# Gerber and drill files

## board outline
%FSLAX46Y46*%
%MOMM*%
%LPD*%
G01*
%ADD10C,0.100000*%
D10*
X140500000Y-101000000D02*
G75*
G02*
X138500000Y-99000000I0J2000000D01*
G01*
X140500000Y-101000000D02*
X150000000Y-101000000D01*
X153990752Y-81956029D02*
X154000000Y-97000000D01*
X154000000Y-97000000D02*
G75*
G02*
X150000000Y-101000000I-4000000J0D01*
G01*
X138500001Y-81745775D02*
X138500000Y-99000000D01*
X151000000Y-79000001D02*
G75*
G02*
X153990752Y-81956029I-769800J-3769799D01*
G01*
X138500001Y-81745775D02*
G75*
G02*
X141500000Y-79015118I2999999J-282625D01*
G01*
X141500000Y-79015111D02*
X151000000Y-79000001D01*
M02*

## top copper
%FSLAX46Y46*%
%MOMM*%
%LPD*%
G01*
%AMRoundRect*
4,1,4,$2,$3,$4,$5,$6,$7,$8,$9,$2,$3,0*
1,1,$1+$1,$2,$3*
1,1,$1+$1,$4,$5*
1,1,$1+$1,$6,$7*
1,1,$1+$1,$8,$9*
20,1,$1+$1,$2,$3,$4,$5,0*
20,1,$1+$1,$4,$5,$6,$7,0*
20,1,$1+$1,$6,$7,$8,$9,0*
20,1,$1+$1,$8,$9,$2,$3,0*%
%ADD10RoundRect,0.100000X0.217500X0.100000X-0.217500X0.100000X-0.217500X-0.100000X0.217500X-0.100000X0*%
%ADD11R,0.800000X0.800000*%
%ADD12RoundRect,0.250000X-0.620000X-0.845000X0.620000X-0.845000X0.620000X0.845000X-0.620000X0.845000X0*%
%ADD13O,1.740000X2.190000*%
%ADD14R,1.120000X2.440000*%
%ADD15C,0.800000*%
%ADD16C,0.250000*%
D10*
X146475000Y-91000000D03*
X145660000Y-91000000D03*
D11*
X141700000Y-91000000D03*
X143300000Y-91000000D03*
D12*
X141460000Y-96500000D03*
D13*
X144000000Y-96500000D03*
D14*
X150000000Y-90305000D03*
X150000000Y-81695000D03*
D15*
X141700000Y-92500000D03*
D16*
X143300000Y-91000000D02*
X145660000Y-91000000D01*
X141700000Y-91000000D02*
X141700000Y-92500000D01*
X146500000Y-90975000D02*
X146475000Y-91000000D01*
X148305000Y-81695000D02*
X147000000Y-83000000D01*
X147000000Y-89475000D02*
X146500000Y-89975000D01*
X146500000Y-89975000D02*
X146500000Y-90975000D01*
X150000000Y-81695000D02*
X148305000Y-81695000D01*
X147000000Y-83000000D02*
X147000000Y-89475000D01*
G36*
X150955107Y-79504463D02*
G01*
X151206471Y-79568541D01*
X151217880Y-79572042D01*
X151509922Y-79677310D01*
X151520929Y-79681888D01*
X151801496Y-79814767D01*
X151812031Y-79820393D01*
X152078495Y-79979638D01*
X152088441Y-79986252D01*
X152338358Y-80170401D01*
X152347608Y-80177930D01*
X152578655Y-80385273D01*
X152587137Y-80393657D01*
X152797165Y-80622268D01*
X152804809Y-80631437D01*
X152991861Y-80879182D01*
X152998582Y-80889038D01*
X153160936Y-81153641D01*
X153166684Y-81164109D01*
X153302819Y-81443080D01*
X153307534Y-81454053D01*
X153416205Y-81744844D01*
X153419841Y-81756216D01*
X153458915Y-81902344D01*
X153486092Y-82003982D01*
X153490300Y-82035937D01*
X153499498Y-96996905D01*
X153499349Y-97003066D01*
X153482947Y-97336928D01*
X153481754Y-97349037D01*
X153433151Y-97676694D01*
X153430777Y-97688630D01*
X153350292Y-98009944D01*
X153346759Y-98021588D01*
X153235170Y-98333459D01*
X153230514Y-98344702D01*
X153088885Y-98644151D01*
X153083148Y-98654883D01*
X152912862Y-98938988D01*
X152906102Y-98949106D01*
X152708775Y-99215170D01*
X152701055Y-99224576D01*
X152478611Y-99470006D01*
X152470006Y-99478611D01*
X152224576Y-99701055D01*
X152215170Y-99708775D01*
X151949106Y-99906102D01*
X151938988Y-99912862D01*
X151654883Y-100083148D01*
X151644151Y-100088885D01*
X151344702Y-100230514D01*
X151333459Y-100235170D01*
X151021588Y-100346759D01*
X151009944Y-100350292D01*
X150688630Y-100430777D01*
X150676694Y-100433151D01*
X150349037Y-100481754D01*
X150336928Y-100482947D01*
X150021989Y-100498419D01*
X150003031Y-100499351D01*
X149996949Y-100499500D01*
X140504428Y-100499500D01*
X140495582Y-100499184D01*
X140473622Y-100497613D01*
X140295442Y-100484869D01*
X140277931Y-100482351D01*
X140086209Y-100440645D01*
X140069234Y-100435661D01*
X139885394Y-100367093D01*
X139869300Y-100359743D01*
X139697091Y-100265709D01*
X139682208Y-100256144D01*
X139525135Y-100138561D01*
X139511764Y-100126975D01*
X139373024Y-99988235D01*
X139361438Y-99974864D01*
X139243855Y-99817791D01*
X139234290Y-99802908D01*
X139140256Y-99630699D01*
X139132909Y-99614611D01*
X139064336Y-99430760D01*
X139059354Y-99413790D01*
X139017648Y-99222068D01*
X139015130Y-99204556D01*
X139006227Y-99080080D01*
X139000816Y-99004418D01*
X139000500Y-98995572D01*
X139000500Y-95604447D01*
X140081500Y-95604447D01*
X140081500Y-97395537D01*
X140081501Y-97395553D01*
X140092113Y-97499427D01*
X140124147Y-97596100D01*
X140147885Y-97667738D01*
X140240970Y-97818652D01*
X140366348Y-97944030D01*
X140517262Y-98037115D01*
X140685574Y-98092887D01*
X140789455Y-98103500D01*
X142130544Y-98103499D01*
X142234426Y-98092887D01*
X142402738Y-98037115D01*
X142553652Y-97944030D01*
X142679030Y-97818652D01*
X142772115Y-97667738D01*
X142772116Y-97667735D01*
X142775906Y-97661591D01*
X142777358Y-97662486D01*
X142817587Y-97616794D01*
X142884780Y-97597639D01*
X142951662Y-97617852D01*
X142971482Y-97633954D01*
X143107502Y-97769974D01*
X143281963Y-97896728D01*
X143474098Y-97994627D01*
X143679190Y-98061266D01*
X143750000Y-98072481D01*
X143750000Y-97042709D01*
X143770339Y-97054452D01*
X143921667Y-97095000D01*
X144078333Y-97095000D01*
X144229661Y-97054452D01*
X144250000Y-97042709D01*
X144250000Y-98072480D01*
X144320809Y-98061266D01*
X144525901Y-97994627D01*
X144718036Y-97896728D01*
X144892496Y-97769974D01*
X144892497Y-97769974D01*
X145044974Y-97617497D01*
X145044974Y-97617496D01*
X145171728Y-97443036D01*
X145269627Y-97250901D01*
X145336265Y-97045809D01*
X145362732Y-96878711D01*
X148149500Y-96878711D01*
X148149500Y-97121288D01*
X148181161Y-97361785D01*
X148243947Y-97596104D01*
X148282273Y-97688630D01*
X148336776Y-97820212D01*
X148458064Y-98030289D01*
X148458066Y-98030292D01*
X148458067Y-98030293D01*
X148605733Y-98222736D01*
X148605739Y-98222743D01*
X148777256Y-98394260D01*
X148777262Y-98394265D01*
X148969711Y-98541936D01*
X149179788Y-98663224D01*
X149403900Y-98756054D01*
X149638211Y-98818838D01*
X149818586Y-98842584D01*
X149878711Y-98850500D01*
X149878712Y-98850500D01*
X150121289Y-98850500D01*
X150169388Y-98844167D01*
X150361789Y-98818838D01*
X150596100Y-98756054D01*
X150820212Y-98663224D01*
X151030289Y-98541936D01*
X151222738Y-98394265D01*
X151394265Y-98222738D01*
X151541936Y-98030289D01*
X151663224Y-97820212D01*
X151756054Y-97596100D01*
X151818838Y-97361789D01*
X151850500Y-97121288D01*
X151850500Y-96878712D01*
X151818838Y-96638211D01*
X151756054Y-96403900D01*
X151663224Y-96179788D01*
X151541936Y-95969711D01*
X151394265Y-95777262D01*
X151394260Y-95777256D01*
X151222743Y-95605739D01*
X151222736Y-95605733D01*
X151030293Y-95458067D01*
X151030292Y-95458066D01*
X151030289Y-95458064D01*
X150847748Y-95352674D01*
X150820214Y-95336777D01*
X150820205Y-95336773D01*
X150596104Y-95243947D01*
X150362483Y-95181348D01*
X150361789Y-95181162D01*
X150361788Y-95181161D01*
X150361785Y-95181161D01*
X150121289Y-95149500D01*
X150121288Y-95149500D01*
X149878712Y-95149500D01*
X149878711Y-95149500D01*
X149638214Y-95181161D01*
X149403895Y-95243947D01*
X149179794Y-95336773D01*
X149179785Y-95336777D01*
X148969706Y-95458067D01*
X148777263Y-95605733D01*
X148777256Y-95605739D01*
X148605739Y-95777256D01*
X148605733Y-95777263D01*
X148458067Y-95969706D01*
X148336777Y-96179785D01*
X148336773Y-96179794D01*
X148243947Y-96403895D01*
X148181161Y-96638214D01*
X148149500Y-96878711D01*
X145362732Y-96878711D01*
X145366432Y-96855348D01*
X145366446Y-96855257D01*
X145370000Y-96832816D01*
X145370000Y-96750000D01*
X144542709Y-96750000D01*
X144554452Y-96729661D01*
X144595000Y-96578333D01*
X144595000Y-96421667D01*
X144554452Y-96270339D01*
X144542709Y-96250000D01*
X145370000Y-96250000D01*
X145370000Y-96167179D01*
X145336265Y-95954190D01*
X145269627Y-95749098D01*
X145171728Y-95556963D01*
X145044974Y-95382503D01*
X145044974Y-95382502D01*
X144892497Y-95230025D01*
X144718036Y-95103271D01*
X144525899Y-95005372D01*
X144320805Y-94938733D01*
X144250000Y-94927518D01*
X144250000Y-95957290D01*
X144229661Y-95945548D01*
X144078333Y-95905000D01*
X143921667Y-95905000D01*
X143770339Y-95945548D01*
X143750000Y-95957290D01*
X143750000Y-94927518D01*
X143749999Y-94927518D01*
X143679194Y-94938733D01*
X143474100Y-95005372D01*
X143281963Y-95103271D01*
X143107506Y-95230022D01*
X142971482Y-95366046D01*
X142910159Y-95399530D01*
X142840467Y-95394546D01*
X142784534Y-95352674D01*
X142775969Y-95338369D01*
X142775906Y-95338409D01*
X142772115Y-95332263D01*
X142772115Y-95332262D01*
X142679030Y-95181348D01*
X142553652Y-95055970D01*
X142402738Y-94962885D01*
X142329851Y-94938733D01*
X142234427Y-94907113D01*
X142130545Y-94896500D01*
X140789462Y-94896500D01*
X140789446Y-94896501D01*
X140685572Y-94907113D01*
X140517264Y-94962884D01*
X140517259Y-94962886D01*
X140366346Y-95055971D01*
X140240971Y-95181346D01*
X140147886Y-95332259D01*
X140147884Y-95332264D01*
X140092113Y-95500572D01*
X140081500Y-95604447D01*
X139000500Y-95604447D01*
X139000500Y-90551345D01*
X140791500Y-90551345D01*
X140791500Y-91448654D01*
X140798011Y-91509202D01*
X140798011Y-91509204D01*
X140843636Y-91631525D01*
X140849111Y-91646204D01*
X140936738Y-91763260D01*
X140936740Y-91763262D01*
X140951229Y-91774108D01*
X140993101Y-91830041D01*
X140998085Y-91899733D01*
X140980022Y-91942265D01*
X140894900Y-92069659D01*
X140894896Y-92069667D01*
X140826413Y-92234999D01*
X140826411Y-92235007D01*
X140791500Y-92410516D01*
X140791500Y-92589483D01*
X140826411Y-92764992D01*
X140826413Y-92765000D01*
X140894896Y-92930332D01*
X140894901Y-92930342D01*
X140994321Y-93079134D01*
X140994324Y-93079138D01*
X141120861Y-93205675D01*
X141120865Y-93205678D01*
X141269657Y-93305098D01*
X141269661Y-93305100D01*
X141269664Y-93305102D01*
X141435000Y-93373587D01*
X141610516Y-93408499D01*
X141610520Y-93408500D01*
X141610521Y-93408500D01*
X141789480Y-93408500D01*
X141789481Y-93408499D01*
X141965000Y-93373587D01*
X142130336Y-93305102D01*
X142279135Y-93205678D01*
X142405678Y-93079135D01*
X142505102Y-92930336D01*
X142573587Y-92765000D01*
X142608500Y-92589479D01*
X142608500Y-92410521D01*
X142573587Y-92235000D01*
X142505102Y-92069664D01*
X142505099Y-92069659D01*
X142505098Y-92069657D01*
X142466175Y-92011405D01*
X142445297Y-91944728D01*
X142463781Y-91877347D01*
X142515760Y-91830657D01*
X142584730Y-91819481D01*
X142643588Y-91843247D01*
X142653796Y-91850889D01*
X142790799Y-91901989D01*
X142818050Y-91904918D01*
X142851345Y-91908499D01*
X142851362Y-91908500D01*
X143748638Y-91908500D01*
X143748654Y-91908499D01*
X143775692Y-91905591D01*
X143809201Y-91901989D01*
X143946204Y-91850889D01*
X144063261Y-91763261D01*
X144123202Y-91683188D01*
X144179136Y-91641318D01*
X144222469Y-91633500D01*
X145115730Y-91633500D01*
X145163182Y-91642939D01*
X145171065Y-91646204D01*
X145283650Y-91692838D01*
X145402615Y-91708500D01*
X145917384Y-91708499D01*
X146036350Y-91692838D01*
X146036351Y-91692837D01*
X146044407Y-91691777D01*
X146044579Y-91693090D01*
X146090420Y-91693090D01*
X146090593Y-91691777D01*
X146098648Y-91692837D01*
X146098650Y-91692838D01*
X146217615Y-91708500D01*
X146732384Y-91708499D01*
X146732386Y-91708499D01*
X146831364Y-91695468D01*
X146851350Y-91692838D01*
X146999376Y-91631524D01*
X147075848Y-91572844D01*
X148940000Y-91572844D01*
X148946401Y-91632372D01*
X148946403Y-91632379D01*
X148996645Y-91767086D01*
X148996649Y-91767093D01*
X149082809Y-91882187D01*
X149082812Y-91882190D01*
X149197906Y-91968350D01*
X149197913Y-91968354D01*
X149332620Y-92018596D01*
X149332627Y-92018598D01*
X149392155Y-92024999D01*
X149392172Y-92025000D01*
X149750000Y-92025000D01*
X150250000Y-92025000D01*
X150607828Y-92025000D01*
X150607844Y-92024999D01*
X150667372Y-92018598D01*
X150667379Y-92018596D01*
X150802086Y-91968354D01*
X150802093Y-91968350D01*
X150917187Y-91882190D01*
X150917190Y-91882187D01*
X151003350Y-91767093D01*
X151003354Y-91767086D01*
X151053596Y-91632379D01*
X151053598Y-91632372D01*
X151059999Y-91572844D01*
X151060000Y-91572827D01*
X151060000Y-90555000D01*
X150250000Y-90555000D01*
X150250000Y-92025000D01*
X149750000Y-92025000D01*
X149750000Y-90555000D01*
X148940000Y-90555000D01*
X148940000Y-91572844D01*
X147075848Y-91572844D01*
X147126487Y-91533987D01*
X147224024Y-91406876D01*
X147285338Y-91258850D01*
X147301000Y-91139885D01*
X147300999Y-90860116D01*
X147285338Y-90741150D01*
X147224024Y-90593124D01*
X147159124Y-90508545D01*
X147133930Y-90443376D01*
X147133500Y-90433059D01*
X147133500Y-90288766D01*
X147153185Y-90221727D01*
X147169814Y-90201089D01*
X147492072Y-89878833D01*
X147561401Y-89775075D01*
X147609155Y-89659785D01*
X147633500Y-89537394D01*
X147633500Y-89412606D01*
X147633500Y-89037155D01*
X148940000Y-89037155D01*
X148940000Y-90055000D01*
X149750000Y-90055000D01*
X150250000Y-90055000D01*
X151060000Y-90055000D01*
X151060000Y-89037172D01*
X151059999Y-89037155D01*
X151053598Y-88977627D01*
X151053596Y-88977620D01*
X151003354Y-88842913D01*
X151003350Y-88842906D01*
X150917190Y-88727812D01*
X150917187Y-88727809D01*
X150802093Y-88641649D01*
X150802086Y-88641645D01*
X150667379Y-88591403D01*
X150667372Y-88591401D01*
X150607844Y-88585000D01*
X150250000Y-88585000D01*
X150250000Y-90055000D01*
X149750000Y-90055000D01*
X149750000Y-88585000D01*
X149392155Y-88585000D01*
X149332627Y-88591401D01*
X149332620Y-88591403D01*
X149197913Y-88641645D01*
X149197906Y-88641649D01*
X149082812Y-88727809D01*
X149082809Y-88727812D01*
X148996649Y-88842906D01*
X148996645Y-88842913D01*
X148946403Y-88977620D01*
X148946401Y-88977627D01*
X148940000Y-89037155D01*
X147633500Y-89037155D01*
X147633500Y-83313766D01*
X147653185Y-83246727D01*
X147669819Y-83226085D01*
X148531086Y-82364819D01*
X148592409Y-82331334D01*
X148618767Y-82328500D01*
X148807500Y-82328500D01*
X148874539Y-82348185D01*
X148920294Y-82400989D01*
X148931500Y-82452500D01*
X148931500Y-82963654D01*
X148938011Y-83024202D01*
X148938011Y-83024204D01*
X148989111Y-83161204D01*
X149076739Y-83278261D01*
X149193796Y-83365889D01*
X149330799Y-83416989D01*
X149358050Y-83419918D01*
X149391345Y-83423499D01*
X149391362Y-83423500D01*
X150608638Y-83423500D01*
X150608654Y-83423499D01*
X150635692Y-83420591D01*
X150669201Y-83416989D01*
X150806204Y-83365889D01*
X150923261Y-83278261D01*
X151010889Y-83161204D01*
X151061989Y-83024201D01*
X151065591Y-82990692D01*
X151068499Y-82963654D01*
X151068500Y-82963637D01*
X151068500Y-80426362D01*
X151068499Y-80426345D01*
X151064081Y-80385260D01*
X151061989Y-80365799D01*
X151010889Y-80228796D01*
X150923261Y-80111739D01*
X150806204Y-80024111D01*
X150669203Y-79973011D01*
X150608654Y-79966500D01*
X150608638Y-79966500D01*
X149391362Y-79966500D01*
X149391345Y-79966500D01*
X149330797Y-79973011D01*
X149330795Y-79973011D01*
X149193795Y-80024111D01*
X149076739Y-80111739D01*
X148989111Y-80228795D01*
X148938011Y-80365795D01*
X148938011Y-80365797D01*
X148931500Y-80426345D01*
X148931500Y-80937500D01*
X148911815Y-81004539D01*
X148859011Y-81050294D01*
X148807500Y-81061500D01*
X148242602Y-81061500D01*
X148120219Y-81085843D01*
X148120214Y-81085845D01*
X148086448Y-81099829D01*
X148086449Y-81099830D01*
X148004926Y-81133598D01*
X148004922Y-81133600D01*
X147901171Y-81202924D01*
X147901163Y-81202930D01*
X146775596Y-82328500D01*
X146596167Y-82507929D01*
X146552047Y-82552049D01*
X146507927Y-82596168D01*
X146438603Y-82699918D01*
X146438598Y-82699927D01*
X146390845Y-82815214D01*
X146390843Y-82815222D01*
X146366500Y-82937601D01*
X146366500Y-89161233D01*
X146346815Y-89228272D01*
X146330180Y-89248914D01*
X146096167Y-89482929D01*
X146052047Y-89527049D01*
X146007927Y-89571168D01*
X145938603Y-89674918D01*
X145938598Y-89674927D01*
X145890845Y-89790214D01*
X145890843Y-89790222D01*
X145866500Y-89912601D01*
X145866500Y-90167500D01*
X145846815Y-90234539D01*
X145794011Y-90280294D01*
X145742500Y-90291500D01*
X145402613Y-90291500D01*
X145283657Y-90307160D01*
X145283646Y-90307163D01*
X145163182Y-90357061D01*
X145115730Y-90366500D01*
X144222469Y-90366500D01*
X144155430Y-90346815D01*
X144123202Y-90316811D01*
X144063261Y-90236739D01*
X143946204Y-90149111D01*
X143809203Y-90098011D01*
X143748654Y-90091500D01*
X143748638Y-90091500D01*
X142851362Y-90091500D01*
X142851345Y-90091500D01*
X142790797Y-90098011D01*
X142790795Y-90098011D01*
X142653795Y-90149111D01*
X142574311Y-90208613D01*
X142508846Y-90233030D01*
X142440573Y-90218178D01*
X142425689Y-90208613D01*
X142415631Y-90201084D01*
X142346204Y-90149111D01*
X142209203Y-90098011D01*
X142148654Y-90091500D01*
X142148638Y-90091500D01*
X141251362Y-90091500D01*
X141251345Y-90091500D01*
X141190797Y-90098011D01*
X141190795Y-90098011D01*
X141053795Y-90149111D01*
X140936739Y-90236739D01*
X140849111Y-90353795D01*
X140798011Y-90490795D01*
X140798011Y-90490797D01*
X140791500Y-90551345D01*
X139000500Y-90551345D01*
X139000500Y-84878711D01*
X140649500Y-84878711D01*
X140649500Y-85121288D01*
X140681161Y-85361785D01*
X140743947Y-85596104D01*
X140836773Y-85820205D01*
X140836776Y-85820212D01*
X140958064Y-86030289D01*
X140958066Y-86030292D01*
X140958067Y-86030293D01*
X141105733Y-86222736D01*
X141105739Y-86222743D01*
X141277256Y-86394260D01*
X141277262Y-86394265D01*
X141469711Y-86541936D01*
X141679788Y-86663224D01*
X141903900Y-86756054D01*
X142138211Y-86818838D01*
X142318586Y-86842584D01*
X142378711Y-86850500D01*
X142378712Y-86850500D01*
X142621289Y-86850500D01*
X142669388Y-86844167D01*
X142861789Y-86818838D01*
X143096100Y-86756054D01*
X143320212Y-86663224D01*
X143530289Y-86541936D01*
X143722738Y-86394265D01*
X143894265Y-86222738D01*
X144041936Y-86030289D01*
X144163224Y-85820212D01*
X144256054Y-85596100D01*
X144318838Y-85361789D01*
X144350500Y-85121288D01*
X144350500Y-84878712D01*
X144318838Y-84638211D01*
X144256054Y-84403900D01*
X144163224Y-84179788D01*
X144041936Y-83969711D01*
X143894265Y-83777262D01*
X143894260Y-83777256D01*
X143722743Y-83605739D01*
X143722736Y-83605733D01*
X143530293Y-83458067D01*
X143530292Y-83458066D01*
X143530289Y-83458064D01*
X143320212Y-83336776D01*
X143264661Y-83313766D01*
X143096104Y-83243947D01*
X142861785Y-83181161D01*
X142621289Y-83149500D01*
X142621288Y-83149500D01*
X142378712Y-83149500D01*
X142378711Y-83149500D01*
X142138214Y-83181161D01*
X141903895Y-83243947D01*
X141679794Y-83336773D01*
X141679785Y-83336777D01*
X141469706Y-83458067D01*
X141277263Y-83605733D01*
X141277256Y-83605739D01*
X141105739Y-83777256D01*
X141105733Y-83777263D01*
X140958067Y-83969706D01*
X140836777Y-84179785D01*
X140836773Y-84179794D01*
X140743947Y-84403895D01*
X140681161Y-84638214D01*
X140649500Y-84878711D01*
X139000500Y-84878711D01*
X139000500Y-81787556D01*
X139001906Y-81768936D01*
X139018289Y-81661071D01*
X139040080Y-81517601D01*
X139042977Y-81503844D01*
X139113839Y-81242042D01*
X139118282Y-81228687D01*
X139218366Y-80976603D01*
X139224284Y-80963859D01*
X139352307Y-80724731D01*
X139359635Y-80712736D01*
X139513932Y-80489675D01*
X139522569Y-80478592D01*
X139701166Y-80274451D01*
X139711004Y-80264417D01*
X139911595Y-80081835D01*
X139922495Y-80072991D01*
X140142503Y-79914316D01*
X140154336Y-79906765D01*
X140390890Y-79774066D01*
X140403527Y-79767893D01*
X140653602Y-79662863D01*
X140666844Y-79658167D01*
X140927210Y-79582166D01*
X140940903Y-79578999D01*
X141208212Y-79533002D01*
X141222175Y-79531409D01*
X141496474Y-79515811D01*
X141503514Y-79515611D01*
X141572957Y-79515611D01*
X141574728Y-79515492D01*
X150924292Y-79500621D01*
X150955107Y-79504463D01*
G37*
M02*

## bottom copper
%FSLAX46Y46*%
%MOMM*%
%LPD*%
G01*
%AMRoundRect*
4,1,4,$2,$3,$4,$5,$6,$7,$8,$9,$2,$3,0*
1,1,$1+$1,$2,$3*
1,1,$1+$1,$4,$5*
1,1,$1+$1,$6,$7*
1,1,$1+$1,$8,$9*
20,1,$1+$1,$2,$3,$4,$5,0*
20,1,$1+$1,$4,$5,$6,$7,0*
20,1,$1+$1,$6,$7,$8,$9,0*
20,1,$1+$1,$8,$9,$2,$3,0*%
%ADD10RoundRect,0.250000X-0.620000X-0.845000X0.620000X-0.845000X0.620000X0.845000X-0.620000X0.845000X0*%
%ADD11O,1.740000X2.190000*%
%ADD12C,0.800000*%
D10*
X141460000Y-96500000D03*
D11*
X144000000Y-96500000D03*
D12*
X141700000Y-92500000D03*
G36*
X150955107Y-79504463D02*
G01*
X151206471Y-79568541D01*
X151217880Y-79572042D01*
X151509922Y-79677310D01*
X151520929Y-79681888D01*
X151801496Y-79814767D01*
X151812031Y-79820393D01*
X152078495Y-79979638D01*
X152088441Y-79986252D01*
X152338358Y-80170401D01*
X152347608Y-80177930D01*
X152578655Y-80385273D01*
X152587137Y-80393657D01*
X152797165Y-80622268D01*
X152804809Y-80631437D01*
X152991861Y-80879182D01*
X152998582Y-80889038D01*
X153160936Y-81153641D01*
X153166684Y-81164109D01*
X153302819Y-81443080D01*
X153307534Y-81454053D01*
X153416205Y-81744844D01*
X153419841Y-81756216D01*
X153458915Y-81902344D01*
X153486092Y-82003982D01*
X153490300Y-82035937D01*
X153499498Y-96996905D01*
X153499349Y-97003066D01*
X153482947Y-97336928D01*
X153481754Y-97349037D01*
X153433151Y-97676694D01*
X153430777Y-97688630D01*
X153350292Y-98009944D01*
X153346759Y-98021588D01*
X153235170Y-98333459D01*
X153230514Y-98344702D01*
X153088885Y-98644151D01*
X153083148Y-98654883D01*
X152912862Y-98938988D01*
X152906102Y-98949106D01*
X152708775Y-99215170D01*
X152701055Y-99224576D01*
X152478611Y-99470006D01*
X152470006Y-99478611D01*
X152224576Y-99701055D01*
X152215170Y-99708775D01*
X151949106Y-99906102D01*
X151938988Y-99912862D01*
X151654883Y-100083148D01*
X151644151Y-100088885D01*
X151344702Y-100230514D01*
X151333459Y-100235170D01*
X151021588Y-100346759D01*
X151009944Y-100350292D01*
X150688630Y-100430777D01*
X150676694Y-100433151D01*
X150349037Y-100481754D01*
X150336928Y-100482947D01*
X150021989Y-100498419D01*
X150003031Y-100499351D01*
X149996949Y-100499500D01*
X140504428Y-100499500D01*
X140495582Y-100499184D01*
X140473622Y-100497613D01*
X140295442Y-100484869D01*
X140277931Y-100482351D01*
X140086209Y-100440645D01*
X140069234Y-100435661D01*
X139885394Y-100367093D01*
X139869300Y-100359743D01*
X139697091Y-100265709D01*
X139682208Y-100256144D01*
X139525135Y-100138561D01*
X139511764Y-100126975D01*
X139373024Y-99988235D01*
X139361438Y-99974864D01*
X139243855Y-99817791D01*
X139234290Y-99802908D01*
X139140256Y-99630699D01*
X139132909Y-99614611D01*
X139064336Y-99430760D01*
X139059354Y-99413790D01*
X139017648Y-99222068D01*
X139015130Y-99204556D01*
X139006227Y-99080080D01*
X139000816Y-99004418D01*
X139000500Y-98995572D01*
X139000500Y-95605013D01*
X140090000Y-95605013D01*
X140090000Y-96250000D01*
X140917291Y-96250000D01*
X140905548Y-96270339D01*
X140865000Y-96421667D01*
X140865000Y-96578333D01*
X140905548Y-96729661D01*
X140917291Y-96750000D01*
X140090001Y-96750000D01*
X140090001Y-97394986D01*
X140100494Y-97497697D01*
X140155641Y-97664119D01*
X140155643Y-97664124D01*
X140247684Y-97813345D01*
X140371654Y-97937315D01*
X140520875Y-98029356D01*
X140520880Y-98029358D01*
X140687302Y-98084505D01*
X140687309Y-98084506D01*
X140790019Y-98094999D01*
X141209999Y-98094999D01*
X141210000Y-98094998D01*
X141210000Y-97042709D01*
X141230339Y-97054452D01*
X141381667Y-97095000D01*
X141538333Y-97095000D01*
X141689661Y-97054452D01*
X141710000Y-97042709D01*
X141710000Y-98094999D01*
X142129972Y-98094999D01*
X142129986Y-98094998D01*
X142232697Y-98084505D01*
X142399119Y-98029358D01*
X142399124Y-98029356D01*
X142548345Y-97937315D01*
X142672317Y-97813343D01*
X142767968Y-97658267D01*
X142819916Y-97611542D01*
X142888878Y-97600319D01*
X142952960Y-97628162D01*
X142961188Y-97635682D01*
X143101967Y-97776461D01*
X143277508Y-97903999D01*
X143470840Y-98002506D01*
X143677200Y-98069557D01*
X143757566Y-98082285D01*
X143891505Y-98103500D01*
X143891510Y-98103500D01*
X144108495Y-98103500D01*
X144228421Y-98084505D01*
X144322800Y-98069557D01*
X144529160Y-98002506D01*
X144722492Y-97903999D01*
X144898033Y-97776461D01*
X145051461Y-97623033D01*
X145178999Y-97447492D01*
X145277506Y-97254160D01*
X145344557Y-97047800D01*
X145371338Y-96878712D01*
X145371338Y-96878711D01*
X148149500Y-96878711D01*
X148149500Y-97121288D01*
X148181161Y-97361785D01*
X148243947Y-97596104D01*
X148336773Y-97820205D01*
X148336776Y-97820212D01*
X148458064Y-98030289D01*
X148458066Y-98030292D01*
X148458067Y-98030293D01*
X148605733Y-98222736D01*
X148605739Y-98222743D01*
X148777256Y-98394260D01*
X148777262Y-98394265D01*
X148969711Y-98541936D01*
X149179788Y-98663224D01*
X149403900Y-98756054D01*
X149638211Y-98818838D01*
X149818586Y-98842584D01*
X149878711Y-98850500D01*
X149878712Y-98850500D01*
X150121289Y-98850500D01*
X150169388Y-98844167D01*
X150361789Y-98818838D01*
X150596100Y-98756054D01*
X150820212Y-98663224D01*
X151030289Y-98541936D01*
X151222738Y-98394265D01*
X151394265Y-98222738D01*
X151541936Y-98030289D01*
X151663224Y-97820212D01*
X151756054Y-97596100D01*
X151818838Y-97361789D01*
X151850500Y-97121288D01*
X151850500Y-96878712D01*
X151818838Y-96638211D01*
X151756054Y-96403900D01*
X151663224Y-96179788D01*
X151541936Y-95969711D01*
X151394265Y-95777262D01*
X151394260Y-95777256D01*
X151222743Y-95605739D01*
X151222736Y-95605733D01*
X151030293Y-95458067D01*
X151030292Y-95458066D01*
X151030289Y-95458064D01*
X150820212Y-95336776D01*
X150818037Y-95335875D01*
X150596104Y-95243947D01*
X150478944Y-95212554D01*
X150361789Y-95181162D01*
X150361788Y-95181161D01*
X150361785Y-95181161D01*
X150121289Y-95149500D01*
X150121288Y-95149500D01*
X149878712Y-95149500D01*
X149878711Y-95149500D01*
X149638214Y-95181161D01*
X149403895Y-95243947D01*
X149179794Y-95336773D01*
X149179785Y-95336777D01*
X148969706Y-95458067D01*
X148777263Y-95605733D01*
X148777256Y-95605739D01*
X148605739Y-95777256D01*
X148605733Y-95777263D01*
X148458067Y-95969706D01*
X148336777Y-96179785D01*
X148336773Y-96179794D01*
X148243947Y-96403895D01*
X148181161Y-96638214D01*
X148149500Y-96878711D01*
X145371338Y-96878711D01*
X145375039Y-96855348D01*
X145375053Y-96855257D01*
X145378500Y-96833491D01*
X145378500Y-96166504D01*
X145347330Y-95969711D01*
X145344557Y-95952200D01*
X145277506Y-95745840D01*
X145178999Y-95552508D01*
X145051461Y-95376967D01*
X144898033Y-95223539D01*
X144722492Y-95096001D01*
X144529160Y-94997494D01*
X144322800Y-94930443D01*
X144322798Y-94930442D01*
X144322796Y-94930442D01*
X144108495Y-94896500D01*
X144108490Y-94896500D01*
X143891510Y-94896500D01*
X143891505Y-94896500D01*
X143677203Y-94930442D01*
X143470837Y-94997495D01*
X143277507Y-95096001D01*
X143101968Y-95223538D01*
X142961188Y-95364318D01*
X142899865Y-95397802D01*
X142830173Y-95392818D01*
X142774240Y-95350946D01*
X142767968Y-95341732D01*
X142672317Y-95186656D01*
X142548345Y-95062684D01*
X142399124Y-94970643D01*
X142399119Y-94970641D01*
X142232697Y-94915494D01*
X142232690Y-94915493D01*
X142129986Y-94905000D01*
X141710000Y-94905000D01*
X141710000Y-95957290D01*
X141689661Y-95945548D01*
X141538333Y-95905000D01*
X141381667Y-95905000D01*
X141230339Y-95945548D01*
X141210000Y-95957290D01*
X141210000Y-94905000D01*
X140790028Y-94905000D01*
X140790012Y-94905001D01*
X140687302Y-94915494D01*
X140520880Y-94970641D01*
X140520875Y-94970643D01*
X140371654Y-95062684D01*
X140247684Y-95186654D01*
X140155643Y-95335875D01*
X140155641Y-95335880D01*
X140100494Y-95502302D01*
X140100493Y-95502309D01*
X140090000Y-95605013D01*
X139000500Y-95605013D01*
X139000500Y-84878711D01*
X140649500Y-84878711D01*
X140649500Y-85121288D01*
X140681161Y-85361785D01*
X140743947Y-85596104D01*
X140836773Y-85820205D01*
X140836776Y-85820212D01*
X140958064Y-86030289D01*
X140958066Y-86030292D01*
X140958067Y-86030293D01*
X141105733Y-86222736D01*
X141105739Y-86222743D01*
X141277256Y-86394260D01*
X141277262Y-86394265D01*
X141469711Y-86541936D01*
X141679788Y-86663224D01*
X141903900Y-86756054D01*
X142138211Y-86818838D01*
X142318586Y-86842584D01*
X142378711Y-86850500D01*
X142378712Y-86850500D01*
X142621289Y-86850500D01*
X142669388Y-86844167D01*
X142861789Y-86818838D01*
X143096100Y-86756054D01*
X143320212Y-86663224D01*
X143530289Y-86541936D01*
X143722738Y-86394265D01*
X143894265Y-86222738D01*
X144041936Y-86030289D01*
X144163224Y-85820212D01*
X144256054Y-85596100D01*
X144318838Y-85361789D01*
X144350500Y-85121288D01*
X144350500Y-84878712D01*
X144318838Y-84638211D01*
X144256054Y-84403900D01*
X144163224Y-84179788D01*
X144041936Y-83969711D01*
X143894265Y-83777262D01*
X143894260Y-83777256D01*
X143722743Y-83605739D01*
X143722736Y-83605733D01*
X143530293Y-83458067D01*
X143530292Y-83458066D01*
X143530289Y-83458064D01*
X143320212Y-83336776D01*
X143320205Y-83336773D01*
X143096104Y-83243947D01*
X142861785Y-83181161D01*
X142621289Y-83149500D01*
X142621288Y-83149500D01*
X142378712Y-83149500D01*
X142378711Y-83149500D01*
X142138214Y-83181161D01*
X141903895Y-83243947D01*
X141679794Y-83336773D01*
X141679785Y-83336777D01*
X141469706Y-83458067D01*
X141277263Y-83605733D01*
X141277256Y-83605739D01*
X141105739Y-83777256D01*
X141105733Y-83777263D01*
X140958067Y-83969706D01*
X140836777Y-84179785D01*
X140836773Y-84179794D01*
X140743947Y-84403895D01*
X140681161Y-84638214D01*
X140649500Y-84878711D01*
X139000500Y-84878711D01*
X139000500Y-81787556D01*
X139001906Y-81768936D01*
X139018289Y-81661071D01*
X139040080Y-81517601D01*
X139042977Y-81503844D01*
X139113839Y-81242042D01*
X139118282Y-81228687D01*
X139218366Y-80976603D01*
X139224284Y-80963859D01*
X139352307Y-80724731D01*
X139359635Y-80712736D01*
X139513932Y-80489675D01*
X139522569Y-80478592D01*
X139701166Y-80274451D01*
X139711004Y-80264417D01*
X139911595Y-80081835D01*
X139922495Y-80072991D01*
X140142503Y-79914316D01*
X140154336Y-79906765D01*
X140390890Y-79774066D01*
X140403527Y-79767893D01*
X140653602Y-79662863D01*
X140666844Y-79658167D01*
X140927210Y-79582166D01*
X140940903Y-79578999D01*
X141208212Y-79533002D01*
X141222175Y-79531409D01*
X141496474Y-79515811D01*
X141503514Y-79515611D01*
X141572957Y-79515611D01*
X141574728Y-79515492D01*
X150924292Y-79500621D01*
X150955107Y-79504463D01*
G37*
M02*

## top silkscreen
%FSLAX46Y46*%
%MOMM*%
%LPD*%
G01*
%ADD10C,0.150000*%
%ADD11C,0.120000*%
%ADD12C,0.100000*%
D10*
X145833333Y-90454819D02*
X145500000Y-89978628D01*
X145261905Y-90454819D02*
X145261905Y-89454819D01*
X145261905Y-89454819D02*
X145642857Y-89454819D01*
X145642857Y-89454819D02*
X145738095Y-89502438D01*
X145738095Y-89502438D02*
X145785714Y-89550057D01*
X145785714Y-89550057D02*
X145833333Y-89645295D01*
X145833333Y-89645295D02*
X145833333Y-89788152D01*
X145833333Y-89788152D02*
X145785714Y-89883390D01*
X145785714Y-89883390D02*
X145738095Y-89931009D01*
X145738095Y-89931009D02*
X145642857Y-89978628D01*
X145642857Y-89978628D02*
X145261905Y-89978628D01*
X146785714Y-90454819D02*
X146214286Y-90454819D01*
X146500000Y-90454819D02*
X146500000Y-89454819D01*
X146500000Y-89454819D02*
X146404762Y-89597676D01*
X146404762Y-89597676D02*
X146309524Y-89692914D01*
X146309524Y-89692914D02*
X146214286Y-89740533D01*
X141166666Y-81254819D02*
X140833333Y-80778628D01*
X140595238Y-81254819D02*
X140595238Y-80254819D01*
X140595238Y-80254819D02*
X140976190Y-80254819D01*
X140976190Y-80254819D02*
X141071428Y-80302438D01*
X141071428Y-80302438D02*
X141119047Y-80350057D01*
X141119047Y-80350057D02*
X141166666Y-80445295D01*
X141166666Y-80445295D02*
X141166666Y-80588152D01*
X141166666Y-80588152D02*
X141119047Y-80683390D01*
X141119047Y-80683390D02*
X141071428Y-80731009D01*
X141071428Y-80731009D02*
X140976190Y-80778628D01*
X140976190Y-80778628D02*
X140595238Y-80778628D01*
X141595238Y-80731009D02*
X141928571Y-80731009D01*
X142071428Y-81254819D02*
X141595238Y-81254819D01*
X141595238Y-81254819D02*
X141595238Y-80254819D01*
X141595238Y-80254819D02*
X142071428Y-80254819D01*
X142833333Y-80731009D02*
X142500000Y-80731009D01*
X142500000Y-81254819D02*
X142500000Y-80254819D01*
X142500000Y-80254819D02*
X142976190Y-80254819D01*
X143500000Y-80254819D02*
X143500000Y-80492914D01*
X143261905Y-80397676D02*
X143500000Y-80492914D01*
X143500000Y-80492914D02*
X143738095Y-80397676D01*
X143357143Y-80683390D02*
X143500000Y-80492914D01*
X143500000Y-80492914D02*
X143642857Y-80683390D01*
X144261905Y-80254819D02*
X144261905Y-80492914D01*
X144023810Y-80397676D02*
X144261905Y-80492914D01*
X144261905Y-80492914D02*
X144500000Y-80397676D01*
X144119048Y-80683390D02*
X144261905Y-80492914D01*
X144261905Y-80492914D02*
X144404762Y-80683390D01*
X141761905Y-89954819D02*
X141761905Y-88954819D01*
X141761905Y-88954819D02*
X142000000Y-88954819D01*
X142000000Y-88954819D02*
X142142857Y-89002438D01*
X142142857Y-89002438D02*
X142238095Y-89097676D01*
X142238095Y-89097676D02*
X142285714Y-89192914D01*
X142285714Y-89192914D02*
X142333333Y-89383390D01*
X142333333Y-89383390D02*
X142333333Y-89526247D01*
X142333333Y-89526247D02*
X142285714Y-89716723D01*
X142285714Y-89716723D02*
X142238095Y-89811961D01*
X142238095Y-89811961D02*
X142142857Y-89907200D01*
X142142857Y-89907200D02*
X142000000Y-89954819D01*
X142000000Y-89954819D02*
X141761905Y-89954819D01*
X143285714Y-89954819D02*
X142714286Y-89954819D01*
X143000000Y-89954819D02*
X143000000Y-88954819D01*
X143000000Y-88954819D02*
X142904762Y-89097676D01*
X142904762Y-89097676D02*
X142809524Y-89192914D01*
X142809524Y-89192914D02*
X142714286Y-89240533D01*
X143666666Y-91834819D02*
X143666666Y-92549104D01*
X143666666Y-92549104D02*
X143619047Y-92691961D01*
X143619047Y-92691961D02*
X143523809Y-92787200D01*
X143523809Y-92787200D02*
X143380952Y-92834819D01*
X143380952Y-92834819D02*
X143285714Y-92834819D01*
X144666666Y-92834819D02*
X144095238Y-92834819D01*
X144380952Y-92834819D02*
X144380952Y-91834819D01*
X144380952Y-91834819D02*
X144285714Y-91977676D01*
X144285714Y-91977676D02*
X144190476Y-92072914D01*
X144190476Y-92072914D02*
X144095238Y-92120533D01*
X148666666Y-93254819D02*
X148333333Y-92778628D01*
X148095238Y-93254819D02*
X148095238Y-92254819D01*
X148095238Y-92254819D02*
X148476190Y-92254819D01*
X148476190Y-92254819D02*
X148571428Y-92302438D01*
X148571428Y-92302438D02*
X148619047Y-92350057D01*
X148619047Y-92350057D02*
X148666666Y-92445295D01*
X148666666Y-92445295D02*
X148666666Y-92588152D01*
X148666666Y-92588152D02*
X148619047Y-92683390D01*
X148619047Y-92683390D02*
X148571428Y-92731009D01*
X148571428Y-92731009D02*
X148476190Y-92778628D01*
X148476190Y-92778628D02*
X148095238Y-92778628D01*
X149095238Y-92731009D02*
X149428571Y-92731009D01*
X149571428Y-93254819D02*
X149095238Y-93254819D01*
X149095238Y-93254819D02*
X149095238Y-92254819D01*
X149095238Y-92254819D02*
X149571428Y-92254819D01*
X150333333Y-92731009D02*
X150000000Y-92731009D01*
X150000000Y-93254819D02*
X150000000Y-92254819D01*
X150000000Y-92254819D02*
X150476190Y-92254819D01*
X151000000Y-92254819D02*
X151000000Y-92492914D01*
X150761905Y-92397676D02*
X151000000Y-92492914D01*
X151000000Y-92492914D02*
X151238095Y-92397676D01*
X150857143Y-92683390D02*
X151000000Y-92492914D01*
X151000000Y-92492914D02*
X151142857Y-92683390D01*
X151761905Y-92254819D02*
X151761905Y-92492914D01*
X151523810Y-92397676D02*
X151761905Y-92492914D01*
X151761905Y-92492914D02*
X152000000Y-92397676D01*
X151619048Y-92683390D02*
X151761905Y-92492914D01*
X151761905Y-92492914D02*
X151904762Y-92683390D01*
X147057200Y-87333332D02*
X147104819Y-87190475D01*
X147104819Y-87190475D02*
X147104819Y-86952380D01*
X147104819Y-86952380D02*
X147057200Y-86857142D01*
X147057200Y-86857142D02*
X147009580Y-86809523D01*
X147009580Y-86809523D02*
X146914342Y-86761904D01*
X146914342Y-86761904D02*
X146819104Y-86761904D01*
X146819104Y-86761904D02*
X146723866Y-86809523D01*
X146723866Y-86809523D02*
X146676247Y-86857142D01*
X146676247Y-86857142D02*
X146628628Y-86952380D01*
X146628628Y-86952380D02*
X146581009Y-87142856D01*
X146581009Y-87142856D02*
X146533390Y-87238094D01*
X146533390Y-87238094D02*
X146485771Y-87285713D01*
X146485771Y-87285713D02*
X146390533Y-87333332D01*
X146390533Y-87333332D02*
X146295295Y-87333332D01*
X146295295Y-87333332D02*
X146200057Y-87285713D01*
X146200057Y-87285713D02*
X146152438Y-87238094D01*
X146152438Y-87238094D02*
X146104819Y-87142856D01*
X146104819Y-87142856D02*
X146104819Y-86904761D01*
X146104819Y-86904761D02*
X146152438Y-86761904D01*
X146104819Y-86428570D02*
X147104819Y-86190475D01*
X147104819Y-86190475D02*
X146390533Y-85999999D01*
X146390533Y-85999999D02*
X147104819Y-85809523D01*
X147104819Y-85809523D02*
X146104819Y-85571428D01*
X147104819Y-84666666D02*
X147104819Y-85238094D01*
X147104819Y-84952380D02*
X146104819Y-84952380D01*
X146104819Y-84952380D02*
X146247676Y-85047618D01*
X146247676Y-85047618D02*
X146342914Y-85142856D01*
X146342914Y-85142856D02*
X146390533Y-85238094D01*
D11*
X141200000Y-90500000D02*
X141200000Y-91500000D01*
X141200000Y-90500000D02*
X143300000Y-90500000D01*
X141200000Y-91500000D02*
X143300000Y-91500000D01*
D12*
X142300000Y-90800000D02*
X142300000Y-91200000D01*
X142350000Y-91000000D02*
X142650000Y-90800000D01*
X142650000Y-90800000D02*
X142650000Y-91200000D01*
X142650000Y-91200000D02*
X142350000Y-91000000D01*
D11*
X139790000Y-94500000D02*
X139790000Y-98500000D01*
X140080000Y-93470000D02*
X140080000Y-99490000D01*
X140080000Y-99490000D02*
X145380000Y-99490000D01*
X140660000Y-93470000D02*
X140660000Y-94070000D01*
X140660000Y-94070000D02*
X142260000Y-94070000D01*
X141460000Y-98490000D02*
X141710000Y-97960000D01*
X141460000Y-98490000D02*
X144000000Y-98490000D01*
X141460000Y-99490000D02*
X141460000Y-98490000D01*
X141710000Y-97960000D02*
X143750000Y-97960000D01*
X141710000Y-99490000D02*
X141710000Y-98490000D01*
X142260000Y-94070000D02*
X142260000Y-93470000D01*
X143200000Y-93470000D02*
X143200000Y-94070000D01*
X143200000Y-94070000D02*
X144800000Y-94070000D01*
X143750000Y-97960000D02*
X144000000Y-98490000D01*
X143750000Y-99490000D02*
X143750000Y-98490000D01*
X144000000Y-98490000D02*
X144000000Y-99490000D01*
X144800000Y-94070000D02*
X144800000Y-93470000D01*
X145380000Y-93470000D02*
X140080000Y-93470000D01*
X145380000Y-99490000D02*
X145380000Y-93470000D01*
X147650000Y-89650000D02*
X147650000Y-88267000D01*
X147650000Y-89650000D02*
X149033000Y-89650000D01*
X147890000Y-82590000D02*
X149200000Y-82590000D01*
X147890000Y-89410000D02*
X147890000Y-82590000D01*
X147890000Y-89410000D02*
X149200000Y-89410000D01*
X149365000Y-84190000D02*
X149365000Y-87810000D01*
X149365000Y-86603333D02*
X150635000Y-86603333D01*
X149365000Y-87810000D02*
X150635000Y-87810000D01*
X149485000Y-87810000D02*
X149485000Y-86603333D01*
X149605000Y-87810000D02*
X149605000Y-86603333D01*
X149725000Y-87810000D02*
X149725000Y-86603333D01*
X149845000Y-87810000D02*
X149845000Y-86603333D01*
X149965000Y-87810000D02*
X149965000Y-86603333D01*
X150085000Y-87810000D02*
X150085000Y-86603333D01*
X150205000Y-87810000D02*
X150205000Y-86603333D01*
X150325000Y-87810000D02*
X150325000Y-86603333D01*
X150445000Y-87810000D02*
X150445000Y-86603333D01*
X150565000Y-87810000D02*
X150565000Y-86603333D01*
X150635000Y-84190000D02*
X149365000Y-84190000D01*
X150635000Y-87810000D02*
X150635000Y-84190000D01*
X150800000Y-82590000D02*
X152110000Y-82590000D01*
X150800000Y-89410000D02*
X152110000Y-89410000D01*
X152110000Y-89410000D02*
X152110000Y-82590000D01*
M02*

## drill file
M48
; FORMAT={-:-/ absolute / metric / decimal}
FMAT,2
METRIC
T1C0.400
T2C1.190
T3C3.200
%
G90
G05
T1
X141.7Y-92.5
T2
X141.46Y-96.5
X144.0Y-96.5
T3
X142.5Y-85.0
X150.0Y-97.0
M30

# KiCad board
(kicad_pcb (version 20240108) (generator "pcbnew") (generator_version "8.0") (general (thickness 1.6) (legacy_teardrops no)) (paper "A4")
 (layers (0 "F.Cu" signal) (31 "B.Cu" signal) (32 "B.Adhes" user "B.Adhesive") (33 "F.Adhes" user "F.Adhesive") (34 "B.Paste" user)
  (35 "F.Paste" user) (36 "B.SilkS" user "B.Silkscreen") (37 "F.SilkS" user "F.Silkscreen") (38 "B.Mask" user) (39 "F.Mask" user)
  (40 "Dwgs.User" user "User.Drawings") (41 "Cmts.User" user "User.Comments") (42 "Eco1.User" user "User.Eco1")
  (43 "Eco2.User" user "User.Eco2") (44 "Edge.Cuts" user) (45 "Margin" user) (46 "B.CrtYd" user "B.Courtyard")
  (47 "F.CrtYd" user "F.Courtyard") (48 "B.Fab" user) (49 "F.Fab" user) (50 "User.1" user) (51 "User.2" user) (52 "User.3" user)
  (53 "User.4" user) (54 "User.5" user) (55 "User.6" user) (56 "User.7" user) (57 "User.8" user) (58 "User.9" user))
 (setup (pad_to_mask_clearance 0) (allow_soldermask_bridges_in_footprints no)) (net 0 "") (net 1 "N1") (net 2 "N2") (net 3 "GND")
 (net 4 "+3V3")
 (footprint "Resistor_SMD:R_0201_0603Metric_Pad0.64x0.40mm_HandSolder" (layer "F.Cu") (at 146.0675 91 180)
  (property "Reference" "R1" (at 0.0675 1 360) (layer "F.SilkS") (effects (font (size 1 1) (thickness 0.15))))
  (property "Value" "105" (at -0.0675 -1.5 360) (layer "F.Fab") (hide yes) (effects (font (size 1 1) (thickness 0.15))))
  (pad "" smd roundrect (at -0.4325 0 180) (size 0.458 0.36) (layers "F.Paste") (roundrect_rratio 0.25))
  (pad "" smd roundrect (at 0.4325 0 180) (size 0.458 0.36) (layers "F.Paste") (roundrect_rratio 0.25))
  (pad "1" smd roundrect (at -0.4075 0 180) (size 0.635 0.4) (layers "F.Cu" "F.Mask") (roundrect_rratio 0.25) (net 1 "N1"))
  (pad "2" smd roundrect (at 0.4075 0 180) (size 0.635 0.4) (layers "F.Cu" "F.Mask") (roundrect_rratio 0.25) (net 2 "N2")))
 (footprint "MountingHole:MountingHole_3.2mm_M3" (layer "F.Cu") (at 142.5 85)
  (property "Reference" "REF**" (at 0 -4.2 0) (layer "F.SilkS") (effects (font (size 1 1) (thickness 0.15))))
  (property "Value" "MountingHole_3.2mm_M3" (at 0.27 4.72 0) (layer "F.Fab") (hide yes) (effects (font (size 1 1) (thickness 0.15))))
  (pad "" np_thru_hole circle (at 0 0) (size 3.2 3.2) (drill 3.2) (layers "*.Cu" "*.Mask")))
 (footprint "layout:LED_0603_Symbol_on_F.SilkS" (layer "F.Cu") (at 142.5 91)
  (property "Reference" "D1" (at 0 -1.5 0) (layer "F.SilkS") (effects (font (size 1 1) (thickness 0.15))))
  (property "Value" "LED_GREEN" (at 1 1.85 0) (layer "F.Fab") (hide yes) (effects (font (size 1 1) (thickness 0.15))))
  (fp_line (start -1.3 -0.5) (end -1.3 0.5) (stroke (width 0.12) (type solid)) (layer "F.SilkS"))
  (fp_line (start -1.3 -0.5) (end 0.8 -0.5) (stroke (width 0.12) (type solid)) (layer "F.SilkS"))
  (fp_line (start -1.3 0.5) (end 0.8 0.5) (stroke (width 0.12) (type solid)) (layer "F.SilkS"))
  (fp_line (start -0.2 -0.2) (end -0.2 0.2) (stroke (width 0.1) (type solid)) (layer "F.SilkS"))
  (fp_line (start -0.15 0) (end 0.15 -0.2) (stroke (width 0.1) (type solid)) (layer "F.SilkS"))
  (fp_line (start 0.15 -0.2) (end 0.15 0.2) (stroke (width 0.1) (type solid)) (layer "F.SilkS"))
  (fp_line (start 0.15 0.2) (end -0.15 0) (stroke (width 0.1) (type solid)) (layer "F.SilkS"))
  (pad "1" smd rect (at -0.8 0 180) (size 0.8 0.8) (layers "F.Cu" "F.Paste" "F.Mask") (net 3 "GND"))
  (pad "2" smd rect (at 0.8 0 180) (size 0.8 0.8) (layers "F.Cu" "F.Paste" "F.Mask") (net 2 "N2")))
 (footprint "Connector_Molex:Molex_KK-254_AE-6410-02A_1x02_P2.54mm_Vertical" (layer "F.Cu") (at 141.46 96.5)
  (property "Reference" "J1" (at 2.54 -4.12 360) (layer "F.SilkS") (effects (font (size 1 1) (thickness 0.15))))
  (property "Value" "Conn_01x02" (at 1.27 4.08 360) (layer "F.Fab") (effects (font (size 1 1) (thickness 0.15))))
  (fp_line (start -1.67 -2) (end -1.67 2) (stroke (width 0.12) (type solid)) (layer "F.SilkS"))
  (fp_line (start -1.38 -3.03) (end -1.38 2.99) (stroke (width 0.12) (type solid)) (layer "F.SilkS"))
  (fp_line (start -1.38 2.99) (end 3.92 2.99) (stroke (width 0.12) (type solid)) (layer "F.SilkS"))
  (fp_line (start -0.8 -3.03) (end -0.8 -2.43) (stroke (width 0.12) (type solid)) (layer "F.SilkS"))
  (fp_line (start -0.8 -2.43) (end 0.8 -2.43) (stroke (width 0.12) (type solid)) (layer "F.SilkS"))
  (fp_line (start 0 1.99) (end 0.25 1.46) (stroke (width 0.12) (type solid)) (layer "F.SilkS"))
  (fp_line (start 0 1.99) (end 2.54 1.99) (stroke (width 0.12) (type solid)) (layer "F.SilkS"))
  (fp_line (start 0 2.99) (end 0 1.99) (stroke (width 0.12) (type solid)) (layer "F.SilkS"))
  (fp_line (start 0.25 1.46) (end 2.29 1.46) (stroke (width 0.12) (type solid)) (layer "F.SilkS"))
  (fp_line (start 0.25 2.99) (end 0.25 1.99) (stroke (width 0.12) (type solid)) (layer "F.SilkS"))
  (fp_line (start 0.8 -2.43) (end 0.8 -3.03) (stroke (width 0.12) (type solid)) (layer "F.SilkS"))
  (fp_line (start 1.74 -3.03) (end 1.74 -2.43) (stroke (width 0.12) (type solid)) (layer "F.SilkS"))
  (fp_line (start 1.74 -2.43) (end 3.34 -2.43) (stroke (width 0.12) (type solid)) (layer "F.SilkS"))
  (fp_line (start 2.29 1.46) (end 2.54 1.99) (stroke (width 0.12) (type solid)) (layer "F.SilkS"))
  (fp_line (start 2.29 2.99) (end 2.29 1.99) (stroke (width 0.12) (type solid)) (layer "F.SilkS"))
  (fp_line (start 2.54 1.99) (end 2.54 2.99) (stroke (width 0.12) (type solid)) (layer "F.SilkS"))
  (fp_line (start 3.34 -2.43) (end 3.34 -3.03) (stroke (width 0.12) (type solid)) (layer "F.SilkS"))
  (fp_line (start 3.92 -3.03) (end -1.38 -3.03) (stroke (width 0.12) (type solid)) (layer "F.SilkS"))
  (fp_line (start 3.92 2.99) (end 3.92 -3.03) (stroke (width 0.12) (type solid)) (layer "F.SilkS"))
  (pad "1" thru_hole roundrect (at 0 0) (size 1.74 2.19) (drill 1.19) (layers "*.Cu" "*.Mask") (remove_unused_layers no)
   (roundrect_rratio 0.143678) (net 3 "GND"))
  (pad "2" thru_hole oval (at 2.54 0) (size 1.74 2.19) (drill 1.19) (layers "*.Cu" "*.Mask") (remove_unused_layers no) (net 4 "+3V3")))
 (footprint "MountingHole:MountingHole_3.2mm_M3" (layer "F.Cu") (at 150 97)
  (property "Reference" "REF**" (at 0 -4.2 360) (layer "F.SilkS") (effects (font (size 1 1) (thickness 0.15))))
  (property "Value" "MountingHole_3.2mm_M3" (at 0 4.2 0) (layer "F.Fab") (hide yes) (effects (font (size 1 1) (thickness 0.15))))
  (pad "" np_thru_hole circle (at 0 0) (size 3.2 3.2) (drill 3.2) (layers "*.Cu" "*.Mask")))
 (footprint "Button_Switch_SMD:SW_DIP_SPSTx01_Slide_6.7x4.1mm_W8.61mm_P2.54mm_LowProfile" (layer "F.Cu") (at 150 86 90)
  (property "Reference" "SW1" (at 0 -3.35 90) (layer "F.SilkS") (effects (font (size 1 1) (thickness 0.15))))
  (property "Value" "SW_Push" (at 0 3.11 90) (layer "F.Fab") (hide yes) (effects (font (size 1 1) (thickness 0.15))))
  (fp_line (start -3.65 -2.35) (end -2.267 -2.35) (stroke (width 0.12) (type solid)) (layer "F.SilkS"))
  (fp_line (start -3.65 -2.35) (end -3.65 -0.967) (stroke (width 0.12) (type solid)) (layer "F.SilkS"))
  (fp_line (start 3.41 -2.11) (end 3.41 -0.8) (stroke (width 0.12) (type solid)) (layer "F.SilkS"))
  (fp_line (start -3.41 -2.11) (end 3.41 -2.11) (stroke (width 0.12) (type solid)) (layer "F.SilkS"))
  (fp_line (start -3.41 -2.11) (end -3.41 -0.8) (stroke (width 0.12) (type solid)) (layer "F.SilkS"))
  (fp_line (start 1.81 -0.635) (end -1.81 -0.635) (stroke (width 0.12) (type solid)) (layer "F.SilkS"))
  (fp_line (start -0.603333 -0.635) (end -0.603333 0.635) (stroke (width 0.12) (type solid)) (layer "F.SilkS"))
  (fp_line (start -1.81 -0.635) (end -1.81 0.635) (stroke (width 0.12) (type solid)) (layer "F.SilkS"))
  (fp_line (start -1.81 -0.515) (end -0.603333 -0.515) (stroke (width 0.12) (type solid)) (layer "F.SilkS"))
  (fp_line (start -1.81 -0.395) (end -0.603333 -0.395) (stroke (width 0.12) (type solid)) (layer "F.SilkS"))
  (fp_line (start -1.81 -0.275) (end -0.603333 -0.275) (stroke (width 0.12) (type solid)) (layer "F.SilkS"))
  (fp_line (start -1.81 -0.155) (end -0.603333 -0.155) (stroke (width 0.12) (type solid)) (layer "F.SilkS"))
  (fp_line (start -1.81 -0.035) (end -0.603333 -0.035) (stroke (width 0.12) (type solid)) (layer "F.SilkS"))
  (fp_line (start -1.81 0.085) (end -0.603333 0.085) (stroke (width 0.12) (type solid)) (layer "F.SilkS"))
  (fp_line (start -1.81 0.205) (end -0.603333 0.205) (stroke (width 0.12) (type solid)) (layer "F.SilkS"))
  (fp_line (start -1.81 0.325) (end -0.603333 0.325) (stroke (width 0.12) (type solid)) (layer "F.SilkS"))
  (fp_line (start -1.81 0.445) (end -0.603333 0.445) (stroke (width 0.12) (type solid)) (layer "F.SilkS"))
  (fp_line (start -1.81 0.565) (end -0.603333 0.565) (stroke (width 0.12) (type solid)) (layer "F.SilkS"))
  (fp_line (start 1.81 0.635) (end 1.81 -0.635) (stroke (width 0.12) (type solid)) (layer "F.SilkS"))
  (fp_line (start -1.81 0.635) (end 1.81 0.635) (stroke (width 0.12) (type solid)) (layer "F.SilkS"))
  (fp_line (start 3.41 0.8) (end 3.41 2.11) (stroke (width 0.12) (type solid)) (layer "F.SilkS"))
  (fp_line (start -3.41 0.8) (end -3.41 2.11) (stroke (width 0.12) (type solid)) (layer "F.SilkS"))
  (fp_line (start -3.41 2.11) (end 3.41 2.11) (stroke (width 0.12) (type solid)) (layer "F.SilkS"))
  (pad "1" smd rect (at -4.305 0 90) (size 2.44 1.12) (layers "F.Cu" "F.Paste" "F.Mask") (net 4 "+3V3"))
  (pad "2" smd rect (at 4.305 0 90) (size 2.44 1.12) (layers "F.Cu" "F.Paste" "F.Mask") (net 1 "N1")))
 (gr_arc (start 140.5 101) (mid 139.085786 100.414214) (end 138.5 99) (stroke (width 0.1) (type default)) (layer "Edge.Cuts"))
 (gr_line (start 140.5 101) (end 150 101) (stroke (width 0.1) (type default)) (layer "Edge.Cuts"))
 (gr_line (start 153.990752 81.956029) (end 154 97) (stroke (width 0.1) (type default)) (layer "Edge.Cuts"))
 (gr_arc (start 154 97) (mid 152.828427 99.828427) (end 150 101) (stroke (width 0.1) (type default)) (layer "Edge.Cuts"))
 (gr_line (start 138.500001 81.745775) (end 138.5 99) (stroke (width 0.1) (type default)) (layer "Edge.Cuts"))
 (gr_arc (start 151 79.000001) (mid 152.934934 80.033294) (end 153.990752 81.956029) (stroke (width 0.1) (type default)) (layer "Edge.Cuts"))
 (gr_arc (start 138.500001 81.745775) (mid 139.471668 79.8) (end 141.5 79.015111) (stroke (width 0.1) (type default)) (layer "Edge.Cuts"))
 (gr_line (start 141.5 79.015111) (end 151 79.000001) (stroke (width 0.1) (type default)) (layer "Edge.Cuts"))
 (segment (start 143.3 91) (end 145.66 91) (width 0.25) (layer "F.Cu") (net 2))
 (segment (start 141.7 91) (end 141.7 92.5) (width 0.25) (layer "F.Cu") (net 3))
 (via (at 141.7 92.5) (size 0.8) (drill 0.4) (layers "F.Cu" "B.Cu") (free yes) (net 3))
 (segment (start 146.5 90.975) (end 146.475 91) (width 0.25) (layer "F.Cu") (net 1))
 (segment (start 148.305 81.695) (end 147 83) (width 0.25) (layer "F.Cu") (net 1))
 (segment (start 147 89.475) (end 146.5 89.975) (width 0.25) (layer "F.Cu") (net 1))
 (segment (start 146.5 89.975) (end 146.5 90.975) (width 0.25) (layer "F.Cu") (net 1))
 (segment (start 150 81.695) (end 148.305 81.695) (width 0.25) (layer "F.Cu") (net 1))
 (segment (start 147 83) (end 147 89.475) (width 0.25) (layer "F.Cu") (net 1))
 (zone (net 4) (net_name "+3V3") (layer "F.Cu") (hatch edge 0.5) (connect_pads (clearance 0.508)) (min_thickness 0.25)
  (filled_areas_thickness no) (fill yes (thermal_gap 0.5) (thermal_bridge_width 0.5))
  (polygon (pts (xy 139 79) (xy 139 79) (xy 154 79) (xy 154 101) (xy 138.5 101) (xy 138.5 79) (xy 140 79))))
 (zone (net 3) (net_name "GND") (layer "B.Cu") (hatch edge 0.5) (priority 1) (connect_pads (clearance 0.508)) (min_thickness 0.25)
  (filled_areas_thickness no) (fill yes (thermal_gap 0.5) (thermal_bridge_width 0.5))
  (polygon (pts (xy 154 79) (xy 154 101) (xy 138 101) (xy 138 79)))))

